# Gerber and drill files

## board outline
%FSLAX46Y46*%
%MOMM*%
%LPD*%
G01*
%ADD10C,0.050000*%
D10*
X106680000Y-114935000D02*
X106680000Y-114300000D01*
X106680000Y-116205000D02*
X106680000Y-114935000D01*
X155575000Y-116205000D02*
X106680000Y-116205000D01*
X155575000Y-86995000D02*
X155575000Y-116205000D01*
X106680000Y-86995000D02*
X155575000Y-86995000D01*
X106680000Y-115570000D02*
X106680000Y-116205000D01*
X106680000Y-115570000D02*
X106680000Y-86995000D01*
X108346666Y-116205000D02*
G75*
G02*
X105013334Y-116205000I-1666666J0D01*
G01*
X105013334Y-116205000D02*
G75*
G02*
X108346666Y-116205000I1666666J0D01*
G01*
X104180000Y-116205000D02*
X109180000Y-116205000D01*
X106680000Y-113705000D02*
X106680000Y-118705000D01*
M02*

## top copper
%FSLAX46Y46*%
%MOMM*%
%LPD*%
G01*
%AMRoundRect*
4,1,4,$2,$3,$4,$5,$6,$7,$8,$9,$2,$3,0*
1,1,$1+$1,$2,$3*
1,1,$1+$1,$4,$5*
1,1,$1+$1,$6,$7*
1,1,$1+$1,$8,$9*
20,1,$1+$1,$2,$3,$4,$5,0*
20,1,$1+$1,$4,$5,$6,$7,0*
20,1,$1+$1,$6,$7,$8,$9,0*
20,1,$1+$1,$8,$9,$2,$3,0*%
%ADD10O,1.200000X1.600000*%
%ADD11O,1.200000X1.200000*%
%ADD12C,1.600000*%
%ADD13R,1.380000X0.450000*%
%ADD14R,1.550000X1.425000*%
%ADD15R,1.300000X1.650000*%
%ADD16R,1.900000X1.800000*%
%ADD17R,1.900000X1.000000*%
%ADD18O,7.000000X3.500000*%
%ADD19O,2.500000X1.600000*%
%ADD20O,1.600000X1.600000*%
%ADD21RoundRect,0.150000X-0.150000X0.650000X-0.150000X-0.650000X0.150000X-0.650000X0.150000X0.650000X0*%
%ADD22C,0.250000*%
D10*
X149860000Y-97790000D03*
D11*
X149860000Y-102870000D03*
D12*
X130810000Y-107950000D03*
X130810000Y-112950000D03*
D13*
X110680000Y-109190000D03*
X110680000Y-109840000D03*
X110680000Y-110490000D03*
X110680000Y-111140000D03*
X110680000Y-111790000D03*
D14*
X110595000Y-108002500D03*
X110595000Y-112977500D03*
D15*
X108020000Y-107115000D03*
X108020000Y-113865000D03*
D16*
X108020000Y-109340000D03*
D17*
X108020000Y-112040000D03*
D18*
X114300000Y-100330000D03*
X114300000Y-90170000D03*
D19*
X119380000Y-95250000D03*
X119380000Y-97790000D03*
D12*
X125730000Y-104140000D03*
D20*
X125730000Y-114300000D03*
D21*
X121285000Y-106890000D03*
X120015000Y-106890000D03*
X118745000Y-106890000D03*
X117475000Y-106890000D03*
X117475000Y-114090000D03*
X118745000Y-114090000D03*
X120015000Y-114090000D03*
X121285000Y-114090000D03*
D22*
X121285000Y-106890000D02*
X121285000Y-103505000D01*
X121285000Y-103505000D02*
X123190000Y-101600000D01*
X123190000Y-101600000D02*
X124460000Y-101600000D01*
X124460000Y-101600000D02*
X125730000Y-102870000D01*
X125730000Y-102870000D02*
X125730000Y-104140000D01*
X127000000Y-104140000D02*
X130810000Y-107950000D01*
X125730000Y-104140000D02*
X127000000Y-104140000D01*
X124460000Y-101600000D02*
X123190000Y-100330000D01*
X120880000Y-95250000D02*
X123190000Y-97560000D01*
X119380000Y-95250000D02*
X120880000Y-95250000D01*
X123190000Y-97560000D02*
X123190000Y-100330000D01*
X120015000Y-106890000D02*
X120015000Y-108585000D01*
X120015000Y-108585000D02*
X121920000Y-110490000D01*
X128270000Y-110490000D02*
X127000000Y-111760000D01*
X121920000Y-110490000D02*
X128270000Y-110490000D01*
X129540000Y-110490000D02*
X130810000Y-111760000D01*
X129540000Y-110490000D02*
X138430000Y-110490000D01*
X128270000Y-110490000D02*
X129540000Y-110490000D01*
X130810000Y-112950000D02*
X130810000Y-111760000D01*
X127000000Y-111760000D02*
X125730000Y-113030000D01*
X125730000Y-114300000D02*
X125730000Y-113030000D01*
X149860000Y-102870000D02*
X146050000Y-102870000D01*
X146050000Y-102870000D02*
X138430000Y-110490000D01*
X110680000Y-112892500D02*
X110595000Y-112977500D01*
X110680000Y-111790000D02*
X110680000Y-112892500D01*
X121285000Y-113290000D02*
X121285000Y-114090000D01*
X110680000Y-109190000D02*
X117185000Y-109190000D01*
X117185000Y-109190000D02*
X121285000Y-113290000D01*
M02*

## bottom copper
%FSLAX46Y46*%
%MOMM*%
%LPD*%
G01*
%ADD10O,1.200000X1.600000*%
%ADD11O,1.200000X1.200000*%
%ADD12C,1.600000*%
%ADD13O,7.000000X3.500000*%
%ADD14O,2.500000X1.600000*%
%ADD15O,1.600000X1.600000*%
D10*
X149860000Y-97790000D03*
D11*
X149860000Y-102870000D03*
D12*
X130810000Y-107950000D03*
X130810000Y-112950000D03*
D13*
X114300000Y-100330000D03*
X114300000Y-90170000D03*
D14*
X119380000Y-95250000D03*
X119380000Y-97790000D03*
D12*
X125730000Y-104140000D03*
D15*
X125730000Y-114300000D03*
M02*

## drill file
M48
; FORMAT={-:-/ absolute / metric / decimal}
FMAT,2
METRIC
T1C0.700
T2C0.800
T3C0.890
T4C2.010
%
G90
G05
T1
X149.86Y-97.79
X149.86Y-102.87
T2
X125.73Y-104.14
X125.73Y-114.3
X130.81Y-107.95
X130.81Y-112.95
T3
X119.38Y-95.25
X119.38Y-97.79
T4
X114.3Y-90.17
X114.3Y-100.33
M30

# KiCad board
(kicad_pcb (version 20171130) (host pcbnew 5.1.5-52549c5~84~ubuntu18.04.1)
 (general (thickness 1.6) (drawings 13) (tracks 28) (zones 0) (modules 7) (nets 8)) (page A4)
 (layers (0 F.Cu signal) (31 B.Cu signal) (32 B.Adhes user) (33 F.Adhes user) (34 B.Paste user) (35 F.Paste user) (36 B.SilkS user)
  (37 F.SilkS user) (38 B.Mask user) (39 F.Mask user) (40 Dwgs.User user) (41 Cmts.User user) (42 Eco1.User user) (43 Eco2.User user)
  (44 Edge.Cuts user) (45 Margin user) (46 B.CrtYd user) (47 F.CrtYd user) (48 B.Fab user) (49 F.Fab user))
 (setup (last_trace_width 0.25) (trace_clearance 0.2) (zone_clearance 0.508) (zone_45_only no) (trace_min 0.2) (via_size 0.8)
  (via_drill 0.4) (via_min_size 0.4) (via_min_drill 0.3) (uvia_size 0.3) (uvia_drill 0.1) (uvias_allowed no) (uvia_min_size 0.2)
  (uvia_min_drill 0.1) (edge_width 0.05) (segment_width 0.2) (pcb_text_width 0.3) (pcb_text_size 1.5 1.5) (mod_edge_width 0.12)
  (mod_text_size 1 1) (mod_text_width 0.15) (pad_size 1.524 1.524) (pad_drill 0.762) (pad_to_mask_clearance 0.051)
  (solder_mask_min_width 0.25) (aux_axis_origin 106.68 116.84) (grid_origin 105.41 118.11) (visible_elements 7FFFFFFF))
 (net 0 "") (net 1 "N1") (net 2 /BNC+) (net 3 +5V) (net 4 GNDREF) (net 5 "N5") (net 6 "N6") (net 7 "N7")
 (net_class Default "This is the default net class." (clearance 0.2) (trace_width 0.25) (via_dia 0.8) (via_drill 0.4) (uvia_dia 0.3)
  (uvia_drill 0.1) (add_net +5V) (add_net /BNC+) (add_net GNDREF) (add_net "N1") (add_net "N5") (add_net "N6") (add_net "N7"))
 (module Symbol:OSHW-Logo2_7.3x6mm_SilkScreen (layer F.Cu) (at 151.13 90.805)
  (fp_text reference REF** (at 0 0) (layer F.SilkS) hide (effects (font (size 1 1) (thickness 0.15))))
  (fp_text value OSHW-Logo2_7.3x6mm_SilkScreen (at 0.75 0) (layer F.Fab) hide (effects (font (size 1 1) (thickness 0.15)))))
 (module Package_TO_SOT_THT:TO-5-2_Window (layer F.Cu) (at 149.86 97.79 270)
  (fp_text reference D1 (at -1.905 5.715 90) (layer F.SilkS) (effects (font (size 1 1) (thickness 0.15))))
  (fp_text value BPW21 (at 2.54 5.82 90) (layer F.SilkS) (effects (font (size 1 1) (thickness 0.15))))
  (pad 1 thru_hole oval (at 0 0 270) (size 1.6 1.2) (drill 0.7) (layers *.Cu *.Mask))
  (pad 2 thru_hole oval (at 5.08 0 270) (size 1.2 1.2) (drill 0.7) (layers *.Cu *.Mask) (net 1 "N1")))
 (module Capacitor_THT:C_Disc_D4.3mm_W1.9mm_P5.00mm (layer F.Cu) (at 130.81 107.95 270)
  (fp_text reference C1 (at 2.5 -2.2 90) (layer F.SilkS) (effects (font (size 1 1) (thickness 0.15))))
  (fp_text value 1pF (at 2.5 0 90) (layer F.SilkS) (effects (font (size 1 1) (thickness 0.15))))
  (pad 1 thru_hole circle (at 0 0 270) (size 1.6 1.6) (drill 0.8) (layers *.Cu *.Mask) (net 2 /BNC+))
  (pad 2 thru_hole circle (at 5 0 270) (size 1.6 1.6) (drill 0.8) (layers *.Cu *.Mask) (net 1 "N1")))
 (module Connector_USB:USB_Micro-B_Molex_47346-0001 (layer F.Cu) (at 109.22 110.49 270)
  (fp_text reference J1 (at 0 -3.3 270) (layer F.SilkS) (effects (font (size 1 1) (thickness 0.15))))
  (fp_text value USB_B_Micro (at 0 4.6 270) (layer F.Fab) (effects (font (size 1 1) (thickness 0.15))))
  (pad 1 smd rect (at -1.3 -1.46 270) (size 0.45 1.38) (layers F.Cu F.Paste F.Mask) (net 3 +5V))
  (pad 2 smd rect (at -0.65 -1.46 270) (size 0.45 1.38) (layers F.Cu F.Paste F.Mask))
  (pad 3 smd rect (at 0 -1.46 270) (size 0.45 1.38) (layers F.Cu F.Paste F.Mask))
  (pad 4 smd rect (at 0.65 -1.46 270) (size 0.45 1.38) (layers F.Cu F.Paste F.Mask))
  (pad 5 smd rect (at 1.3 -1.46 270) (size 0.45 1.38) (layers F.Cu F.Paste F.Mask) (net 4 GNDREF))
  (pad 6 smd rect (at -2.4875 -1.375 270) (size 1.425 1.55) (layers F.Cu F.Paste F.Mask))
  (pad 6 smd rect (at 2.4875 -1.375 270) (size 1.425 1.55) (layers F.Cu F.Paste F.Mask) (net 4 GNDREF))
  (pad 6 smd rect (at -3.375 1.2 270) (size 1.65 1.3) (layers F.Cu F.Paste F.Mask))
  (pad 6 smd rect (at 3.375 1.2 270) (size 1.65 1.3) (layers F.Cu F.Paste F.Mask))
  (pad 6 smd rect (at -1.15 1.2 270) (size 1.8 1.9) (layers F.Cu F.Paste F.Mask))
  (pad 6 smd rect (at 1.55 1.2 270) (size 1 1.9) (layers F.Cu F.Paste F.Mask)))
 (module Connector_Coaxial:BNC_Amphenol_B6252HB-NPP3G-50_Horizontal (layer F.Cu) (at 119.38 95.25 90)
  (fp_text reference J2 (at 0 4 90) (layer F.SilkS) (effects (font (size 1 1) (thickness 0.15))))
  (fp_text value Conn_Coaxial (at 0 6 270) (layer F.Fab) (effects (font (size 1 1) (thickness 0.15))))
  (pad 2 thru_hole oval (at -5.08 -5.08 90) (size 3.5 7) (drill 2.01) (layers *.Cu *.Mask))
  (pad 2 thru_hole oval (at 5.08 -5.08 90) (size 3.5 7) (drill 2.01) (layers *.Cu *.Mask))
  (pad 1 thru_hole oval (at 0 0 90) (size 1.6 2.5) (drill 0.89) (layers *.Cu *.Mask) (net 2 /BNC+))
  (pad 2 thru_hole oval (at -2.54 0 90) (size 1.6 2.5) (drill 0.89) (layers *.Cu *.Mask)))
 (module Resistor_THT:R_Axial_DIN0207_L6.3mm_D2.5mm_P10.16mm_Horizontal (layer F.Cu) (at 125.73 104.14 270)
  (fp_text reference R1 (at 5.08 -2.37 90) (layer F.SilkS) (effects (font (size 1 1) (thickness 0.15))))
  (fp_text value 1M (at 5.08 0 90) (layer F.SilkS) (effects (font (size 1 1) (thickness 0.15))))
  (pad 1 thru_hole circle (at 0 0 270) (size 1.6 1.6) (drill 0.8) (layers *.Cu *.Mask) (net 2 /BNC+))
  (pad 2 thru_hole oval (at 10.16 0 270) (size 1.6 1.6) (drill 0.8) (layers *.Cu *.Mask) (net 1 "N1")))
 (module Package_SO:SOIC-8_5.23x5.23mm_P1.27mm (layer F.Cu) (at 119.38 110.49 270)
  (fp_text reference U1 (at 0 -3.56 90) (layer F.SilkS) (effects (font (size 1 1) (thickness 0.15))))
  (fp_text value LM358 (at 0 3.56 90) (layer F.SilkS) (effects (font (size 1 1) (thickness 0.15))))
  (pad 1 smd roundrect (at -3.6 -1.905 270) (size 1.6 0.6) (layers F.Cu F.Paste F.Mask) (roundrect_rratio 0.25) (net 2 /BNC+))
  (pad 2 smd roundrect (at -3.6 -0.635 270) (size 1.6 0.6) (layers F.Cu F.Paste F.Mask) (roundrect_rratio 0.25) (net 1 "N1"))
  (pad 3 smd roundrect (at -3.6 0.635 270) (size 1.6 0.6) (layers F.Cu F.Paste F.Mask) (roundrect_rratio 0.25))
  (pad 4 smd roundrect (at -3.6 1.905 270) (size 1.6 0.6) (layers F.Cu F.Paste F.Mask) (roundrect_rratio 0.25))
  (pad 5 smd roundrect (at 3.6 1.905 270) (size 1.6 0.6) (layers F.Cu F.Paste F.Mask) (roundrect_rratio 0.25))
  (pad 6 smd roundrect (at 3.6 0.635 270) (size 1.6 0.6) (layers F.Cu F.Paste F.Mask) (roundrect_rratio 0.25))
  (pad 7 smd roundrect (at 3.6 -0.635 270) (size 1.6 0.6) (layers F.Cu F.Paste F.Mask) (roundrect_rratio 0.25))
  (pad 8 smd roundrect (at 3.6 -1.905 270) (size 1.6 0.6) (layers F.Cu F.Paste F.Mask) (roundrect_rratio 0.25) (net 3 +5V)))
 (gr_line (start 106.68 114.935) (end 106.68 114.3) (layer Edge.Cuts) (width 0.05))
 (gr_line (start 106.68 116.205) (end 106.68 114.935) (layer Edge.Cuts) (width 0.05))
 (gr_line (start 155.575 116.205) (end 106.68 116.205) (layer Edge.Cuts) (width 0.05))
 (gr_line (start 155.575 86.995) (end 155.575 116.205) (layer Edge.Cuts) (width 0.05))
 (gr_line (start 106.68 86.995) (end 155.575 86.995) (layer Edge.Cuts) (width 0.05))
 (gr_line (start 106.68 115.57) (end 106.68 116.205) (layer Edge.Cuts) (width 0.05))
 (gr_line (start 106.68 115.57) (end 106.68 86.995) (layer Edge.Cuts) (width 0.05))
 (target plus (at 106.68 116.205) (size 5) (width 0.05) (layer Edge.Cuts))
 (segment (start 121.285 106.89) (end 121.285 103.505) (width 0.25) (layer F.Cu) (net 2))
 (segment (start 121.285 103.505) (end 123.19 101.6) (width 0.25) (layer F.Cu) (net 2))
 (segment (start 123.19 101.6) (end 124.46 101.6) (width 0.25) (layer F.Cu) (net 2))
 (segment (start 124.46 101.6) (end 125.73 102.87) (width 0.25) (layer F.Cu) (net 2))
 (segment (start 125.73 102.87) (end 125.73 104.14) (width 0.25) (layer F.Cu) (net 2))
 (segment (start 127 104.14) (end 130.81 107.95) (width 0.25) (layer F.Cu) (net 2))
 (segment (start 125.73 104.14) (end 127 104.14) (width 0.25) (layer F.Cu) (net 2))
 (segment (start 124.46 101.6) (end 123.19 100.33) (width 0.25) (layer F.Cu) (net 2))
 (segment (start 120.88 95.25) (end 123.19 97.56) (width 0.25) (layer F.Cu) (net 2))
 (segment (start 119.38 95.25) (end 120.88 95.25) (width 0.25) (layer F.Cu) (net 2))
 (segment (start 123.19 97.56) (end 123.19 100.33) (width 0.25) (layer F.Cu) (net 2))
 (segment (start 120.015 106.89) (end 120.015 108.585) (width 0.25) (layer F.Cu) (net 1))
 (segment (start 120.015 108.585) (end 121.92 110.49) (width 0.25) (layer F.Cu) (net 1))
 (segment (start 128.27 110.49) (end 127 111.76) (width 0.25) (layer F.Cu) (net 1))
 (segment (start 121.92 110.49) (end 128.27 110.49) (width 0.25) (layer F.Cu) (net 1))
 (segment (start 129.54 110.49) (end 130.81 111.76) (width 0.25) (layer F.Cu) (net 1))
 (segment (start 129.54 110.49) (end 138.43 110.49) (width 0.25) (layer F.Cu) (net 1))
 (segment (start 128.27 110.49) (end 129.54 110.49) (width 0.25) (layer F.Cu) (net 1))
 (segment (start 130.81 112.95) (end 130.81 111.76) (width 0.25) (layer F.Cu) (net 1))
 (segment (start 127 111.76) (end 125.73 113.03) (width 0.25) (layer F.Cu) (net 1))
 (segment (start 125.73 114.3) (end 125.73 113.03) (width 0.25) (layer F.Cu) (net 1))
 (segment (start 149.86 102.87) (end 146.05 102.87) (width 0.25) (layer F.Cu) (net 1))
 (segment (start 146.05 102.87) (end 138.43 110.49) (width 0.25) (layer F.Cu) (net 1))
 (segment (start 110.68 112.8925) (end 110.595 112.9775) (width 0.25) (layer F.Cu) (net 4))
 (segment (start 110.68 111.79) (end 110.68 112.8925) (width 0.25) (layer F.Cu) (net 4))
 (segment (start 121.285 113.29) (end 121.285 114.09) (width 0.25) (layer F.Cu) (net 3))
 (segment (start 110.68 109.19) (end 117.185 109.19) (width 0.25) (layer F.Cu) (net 3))
 (segment (start 117.185 109.19) (end 121.285 113.29) (width 0.25) (layer F.Cu) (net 3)))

